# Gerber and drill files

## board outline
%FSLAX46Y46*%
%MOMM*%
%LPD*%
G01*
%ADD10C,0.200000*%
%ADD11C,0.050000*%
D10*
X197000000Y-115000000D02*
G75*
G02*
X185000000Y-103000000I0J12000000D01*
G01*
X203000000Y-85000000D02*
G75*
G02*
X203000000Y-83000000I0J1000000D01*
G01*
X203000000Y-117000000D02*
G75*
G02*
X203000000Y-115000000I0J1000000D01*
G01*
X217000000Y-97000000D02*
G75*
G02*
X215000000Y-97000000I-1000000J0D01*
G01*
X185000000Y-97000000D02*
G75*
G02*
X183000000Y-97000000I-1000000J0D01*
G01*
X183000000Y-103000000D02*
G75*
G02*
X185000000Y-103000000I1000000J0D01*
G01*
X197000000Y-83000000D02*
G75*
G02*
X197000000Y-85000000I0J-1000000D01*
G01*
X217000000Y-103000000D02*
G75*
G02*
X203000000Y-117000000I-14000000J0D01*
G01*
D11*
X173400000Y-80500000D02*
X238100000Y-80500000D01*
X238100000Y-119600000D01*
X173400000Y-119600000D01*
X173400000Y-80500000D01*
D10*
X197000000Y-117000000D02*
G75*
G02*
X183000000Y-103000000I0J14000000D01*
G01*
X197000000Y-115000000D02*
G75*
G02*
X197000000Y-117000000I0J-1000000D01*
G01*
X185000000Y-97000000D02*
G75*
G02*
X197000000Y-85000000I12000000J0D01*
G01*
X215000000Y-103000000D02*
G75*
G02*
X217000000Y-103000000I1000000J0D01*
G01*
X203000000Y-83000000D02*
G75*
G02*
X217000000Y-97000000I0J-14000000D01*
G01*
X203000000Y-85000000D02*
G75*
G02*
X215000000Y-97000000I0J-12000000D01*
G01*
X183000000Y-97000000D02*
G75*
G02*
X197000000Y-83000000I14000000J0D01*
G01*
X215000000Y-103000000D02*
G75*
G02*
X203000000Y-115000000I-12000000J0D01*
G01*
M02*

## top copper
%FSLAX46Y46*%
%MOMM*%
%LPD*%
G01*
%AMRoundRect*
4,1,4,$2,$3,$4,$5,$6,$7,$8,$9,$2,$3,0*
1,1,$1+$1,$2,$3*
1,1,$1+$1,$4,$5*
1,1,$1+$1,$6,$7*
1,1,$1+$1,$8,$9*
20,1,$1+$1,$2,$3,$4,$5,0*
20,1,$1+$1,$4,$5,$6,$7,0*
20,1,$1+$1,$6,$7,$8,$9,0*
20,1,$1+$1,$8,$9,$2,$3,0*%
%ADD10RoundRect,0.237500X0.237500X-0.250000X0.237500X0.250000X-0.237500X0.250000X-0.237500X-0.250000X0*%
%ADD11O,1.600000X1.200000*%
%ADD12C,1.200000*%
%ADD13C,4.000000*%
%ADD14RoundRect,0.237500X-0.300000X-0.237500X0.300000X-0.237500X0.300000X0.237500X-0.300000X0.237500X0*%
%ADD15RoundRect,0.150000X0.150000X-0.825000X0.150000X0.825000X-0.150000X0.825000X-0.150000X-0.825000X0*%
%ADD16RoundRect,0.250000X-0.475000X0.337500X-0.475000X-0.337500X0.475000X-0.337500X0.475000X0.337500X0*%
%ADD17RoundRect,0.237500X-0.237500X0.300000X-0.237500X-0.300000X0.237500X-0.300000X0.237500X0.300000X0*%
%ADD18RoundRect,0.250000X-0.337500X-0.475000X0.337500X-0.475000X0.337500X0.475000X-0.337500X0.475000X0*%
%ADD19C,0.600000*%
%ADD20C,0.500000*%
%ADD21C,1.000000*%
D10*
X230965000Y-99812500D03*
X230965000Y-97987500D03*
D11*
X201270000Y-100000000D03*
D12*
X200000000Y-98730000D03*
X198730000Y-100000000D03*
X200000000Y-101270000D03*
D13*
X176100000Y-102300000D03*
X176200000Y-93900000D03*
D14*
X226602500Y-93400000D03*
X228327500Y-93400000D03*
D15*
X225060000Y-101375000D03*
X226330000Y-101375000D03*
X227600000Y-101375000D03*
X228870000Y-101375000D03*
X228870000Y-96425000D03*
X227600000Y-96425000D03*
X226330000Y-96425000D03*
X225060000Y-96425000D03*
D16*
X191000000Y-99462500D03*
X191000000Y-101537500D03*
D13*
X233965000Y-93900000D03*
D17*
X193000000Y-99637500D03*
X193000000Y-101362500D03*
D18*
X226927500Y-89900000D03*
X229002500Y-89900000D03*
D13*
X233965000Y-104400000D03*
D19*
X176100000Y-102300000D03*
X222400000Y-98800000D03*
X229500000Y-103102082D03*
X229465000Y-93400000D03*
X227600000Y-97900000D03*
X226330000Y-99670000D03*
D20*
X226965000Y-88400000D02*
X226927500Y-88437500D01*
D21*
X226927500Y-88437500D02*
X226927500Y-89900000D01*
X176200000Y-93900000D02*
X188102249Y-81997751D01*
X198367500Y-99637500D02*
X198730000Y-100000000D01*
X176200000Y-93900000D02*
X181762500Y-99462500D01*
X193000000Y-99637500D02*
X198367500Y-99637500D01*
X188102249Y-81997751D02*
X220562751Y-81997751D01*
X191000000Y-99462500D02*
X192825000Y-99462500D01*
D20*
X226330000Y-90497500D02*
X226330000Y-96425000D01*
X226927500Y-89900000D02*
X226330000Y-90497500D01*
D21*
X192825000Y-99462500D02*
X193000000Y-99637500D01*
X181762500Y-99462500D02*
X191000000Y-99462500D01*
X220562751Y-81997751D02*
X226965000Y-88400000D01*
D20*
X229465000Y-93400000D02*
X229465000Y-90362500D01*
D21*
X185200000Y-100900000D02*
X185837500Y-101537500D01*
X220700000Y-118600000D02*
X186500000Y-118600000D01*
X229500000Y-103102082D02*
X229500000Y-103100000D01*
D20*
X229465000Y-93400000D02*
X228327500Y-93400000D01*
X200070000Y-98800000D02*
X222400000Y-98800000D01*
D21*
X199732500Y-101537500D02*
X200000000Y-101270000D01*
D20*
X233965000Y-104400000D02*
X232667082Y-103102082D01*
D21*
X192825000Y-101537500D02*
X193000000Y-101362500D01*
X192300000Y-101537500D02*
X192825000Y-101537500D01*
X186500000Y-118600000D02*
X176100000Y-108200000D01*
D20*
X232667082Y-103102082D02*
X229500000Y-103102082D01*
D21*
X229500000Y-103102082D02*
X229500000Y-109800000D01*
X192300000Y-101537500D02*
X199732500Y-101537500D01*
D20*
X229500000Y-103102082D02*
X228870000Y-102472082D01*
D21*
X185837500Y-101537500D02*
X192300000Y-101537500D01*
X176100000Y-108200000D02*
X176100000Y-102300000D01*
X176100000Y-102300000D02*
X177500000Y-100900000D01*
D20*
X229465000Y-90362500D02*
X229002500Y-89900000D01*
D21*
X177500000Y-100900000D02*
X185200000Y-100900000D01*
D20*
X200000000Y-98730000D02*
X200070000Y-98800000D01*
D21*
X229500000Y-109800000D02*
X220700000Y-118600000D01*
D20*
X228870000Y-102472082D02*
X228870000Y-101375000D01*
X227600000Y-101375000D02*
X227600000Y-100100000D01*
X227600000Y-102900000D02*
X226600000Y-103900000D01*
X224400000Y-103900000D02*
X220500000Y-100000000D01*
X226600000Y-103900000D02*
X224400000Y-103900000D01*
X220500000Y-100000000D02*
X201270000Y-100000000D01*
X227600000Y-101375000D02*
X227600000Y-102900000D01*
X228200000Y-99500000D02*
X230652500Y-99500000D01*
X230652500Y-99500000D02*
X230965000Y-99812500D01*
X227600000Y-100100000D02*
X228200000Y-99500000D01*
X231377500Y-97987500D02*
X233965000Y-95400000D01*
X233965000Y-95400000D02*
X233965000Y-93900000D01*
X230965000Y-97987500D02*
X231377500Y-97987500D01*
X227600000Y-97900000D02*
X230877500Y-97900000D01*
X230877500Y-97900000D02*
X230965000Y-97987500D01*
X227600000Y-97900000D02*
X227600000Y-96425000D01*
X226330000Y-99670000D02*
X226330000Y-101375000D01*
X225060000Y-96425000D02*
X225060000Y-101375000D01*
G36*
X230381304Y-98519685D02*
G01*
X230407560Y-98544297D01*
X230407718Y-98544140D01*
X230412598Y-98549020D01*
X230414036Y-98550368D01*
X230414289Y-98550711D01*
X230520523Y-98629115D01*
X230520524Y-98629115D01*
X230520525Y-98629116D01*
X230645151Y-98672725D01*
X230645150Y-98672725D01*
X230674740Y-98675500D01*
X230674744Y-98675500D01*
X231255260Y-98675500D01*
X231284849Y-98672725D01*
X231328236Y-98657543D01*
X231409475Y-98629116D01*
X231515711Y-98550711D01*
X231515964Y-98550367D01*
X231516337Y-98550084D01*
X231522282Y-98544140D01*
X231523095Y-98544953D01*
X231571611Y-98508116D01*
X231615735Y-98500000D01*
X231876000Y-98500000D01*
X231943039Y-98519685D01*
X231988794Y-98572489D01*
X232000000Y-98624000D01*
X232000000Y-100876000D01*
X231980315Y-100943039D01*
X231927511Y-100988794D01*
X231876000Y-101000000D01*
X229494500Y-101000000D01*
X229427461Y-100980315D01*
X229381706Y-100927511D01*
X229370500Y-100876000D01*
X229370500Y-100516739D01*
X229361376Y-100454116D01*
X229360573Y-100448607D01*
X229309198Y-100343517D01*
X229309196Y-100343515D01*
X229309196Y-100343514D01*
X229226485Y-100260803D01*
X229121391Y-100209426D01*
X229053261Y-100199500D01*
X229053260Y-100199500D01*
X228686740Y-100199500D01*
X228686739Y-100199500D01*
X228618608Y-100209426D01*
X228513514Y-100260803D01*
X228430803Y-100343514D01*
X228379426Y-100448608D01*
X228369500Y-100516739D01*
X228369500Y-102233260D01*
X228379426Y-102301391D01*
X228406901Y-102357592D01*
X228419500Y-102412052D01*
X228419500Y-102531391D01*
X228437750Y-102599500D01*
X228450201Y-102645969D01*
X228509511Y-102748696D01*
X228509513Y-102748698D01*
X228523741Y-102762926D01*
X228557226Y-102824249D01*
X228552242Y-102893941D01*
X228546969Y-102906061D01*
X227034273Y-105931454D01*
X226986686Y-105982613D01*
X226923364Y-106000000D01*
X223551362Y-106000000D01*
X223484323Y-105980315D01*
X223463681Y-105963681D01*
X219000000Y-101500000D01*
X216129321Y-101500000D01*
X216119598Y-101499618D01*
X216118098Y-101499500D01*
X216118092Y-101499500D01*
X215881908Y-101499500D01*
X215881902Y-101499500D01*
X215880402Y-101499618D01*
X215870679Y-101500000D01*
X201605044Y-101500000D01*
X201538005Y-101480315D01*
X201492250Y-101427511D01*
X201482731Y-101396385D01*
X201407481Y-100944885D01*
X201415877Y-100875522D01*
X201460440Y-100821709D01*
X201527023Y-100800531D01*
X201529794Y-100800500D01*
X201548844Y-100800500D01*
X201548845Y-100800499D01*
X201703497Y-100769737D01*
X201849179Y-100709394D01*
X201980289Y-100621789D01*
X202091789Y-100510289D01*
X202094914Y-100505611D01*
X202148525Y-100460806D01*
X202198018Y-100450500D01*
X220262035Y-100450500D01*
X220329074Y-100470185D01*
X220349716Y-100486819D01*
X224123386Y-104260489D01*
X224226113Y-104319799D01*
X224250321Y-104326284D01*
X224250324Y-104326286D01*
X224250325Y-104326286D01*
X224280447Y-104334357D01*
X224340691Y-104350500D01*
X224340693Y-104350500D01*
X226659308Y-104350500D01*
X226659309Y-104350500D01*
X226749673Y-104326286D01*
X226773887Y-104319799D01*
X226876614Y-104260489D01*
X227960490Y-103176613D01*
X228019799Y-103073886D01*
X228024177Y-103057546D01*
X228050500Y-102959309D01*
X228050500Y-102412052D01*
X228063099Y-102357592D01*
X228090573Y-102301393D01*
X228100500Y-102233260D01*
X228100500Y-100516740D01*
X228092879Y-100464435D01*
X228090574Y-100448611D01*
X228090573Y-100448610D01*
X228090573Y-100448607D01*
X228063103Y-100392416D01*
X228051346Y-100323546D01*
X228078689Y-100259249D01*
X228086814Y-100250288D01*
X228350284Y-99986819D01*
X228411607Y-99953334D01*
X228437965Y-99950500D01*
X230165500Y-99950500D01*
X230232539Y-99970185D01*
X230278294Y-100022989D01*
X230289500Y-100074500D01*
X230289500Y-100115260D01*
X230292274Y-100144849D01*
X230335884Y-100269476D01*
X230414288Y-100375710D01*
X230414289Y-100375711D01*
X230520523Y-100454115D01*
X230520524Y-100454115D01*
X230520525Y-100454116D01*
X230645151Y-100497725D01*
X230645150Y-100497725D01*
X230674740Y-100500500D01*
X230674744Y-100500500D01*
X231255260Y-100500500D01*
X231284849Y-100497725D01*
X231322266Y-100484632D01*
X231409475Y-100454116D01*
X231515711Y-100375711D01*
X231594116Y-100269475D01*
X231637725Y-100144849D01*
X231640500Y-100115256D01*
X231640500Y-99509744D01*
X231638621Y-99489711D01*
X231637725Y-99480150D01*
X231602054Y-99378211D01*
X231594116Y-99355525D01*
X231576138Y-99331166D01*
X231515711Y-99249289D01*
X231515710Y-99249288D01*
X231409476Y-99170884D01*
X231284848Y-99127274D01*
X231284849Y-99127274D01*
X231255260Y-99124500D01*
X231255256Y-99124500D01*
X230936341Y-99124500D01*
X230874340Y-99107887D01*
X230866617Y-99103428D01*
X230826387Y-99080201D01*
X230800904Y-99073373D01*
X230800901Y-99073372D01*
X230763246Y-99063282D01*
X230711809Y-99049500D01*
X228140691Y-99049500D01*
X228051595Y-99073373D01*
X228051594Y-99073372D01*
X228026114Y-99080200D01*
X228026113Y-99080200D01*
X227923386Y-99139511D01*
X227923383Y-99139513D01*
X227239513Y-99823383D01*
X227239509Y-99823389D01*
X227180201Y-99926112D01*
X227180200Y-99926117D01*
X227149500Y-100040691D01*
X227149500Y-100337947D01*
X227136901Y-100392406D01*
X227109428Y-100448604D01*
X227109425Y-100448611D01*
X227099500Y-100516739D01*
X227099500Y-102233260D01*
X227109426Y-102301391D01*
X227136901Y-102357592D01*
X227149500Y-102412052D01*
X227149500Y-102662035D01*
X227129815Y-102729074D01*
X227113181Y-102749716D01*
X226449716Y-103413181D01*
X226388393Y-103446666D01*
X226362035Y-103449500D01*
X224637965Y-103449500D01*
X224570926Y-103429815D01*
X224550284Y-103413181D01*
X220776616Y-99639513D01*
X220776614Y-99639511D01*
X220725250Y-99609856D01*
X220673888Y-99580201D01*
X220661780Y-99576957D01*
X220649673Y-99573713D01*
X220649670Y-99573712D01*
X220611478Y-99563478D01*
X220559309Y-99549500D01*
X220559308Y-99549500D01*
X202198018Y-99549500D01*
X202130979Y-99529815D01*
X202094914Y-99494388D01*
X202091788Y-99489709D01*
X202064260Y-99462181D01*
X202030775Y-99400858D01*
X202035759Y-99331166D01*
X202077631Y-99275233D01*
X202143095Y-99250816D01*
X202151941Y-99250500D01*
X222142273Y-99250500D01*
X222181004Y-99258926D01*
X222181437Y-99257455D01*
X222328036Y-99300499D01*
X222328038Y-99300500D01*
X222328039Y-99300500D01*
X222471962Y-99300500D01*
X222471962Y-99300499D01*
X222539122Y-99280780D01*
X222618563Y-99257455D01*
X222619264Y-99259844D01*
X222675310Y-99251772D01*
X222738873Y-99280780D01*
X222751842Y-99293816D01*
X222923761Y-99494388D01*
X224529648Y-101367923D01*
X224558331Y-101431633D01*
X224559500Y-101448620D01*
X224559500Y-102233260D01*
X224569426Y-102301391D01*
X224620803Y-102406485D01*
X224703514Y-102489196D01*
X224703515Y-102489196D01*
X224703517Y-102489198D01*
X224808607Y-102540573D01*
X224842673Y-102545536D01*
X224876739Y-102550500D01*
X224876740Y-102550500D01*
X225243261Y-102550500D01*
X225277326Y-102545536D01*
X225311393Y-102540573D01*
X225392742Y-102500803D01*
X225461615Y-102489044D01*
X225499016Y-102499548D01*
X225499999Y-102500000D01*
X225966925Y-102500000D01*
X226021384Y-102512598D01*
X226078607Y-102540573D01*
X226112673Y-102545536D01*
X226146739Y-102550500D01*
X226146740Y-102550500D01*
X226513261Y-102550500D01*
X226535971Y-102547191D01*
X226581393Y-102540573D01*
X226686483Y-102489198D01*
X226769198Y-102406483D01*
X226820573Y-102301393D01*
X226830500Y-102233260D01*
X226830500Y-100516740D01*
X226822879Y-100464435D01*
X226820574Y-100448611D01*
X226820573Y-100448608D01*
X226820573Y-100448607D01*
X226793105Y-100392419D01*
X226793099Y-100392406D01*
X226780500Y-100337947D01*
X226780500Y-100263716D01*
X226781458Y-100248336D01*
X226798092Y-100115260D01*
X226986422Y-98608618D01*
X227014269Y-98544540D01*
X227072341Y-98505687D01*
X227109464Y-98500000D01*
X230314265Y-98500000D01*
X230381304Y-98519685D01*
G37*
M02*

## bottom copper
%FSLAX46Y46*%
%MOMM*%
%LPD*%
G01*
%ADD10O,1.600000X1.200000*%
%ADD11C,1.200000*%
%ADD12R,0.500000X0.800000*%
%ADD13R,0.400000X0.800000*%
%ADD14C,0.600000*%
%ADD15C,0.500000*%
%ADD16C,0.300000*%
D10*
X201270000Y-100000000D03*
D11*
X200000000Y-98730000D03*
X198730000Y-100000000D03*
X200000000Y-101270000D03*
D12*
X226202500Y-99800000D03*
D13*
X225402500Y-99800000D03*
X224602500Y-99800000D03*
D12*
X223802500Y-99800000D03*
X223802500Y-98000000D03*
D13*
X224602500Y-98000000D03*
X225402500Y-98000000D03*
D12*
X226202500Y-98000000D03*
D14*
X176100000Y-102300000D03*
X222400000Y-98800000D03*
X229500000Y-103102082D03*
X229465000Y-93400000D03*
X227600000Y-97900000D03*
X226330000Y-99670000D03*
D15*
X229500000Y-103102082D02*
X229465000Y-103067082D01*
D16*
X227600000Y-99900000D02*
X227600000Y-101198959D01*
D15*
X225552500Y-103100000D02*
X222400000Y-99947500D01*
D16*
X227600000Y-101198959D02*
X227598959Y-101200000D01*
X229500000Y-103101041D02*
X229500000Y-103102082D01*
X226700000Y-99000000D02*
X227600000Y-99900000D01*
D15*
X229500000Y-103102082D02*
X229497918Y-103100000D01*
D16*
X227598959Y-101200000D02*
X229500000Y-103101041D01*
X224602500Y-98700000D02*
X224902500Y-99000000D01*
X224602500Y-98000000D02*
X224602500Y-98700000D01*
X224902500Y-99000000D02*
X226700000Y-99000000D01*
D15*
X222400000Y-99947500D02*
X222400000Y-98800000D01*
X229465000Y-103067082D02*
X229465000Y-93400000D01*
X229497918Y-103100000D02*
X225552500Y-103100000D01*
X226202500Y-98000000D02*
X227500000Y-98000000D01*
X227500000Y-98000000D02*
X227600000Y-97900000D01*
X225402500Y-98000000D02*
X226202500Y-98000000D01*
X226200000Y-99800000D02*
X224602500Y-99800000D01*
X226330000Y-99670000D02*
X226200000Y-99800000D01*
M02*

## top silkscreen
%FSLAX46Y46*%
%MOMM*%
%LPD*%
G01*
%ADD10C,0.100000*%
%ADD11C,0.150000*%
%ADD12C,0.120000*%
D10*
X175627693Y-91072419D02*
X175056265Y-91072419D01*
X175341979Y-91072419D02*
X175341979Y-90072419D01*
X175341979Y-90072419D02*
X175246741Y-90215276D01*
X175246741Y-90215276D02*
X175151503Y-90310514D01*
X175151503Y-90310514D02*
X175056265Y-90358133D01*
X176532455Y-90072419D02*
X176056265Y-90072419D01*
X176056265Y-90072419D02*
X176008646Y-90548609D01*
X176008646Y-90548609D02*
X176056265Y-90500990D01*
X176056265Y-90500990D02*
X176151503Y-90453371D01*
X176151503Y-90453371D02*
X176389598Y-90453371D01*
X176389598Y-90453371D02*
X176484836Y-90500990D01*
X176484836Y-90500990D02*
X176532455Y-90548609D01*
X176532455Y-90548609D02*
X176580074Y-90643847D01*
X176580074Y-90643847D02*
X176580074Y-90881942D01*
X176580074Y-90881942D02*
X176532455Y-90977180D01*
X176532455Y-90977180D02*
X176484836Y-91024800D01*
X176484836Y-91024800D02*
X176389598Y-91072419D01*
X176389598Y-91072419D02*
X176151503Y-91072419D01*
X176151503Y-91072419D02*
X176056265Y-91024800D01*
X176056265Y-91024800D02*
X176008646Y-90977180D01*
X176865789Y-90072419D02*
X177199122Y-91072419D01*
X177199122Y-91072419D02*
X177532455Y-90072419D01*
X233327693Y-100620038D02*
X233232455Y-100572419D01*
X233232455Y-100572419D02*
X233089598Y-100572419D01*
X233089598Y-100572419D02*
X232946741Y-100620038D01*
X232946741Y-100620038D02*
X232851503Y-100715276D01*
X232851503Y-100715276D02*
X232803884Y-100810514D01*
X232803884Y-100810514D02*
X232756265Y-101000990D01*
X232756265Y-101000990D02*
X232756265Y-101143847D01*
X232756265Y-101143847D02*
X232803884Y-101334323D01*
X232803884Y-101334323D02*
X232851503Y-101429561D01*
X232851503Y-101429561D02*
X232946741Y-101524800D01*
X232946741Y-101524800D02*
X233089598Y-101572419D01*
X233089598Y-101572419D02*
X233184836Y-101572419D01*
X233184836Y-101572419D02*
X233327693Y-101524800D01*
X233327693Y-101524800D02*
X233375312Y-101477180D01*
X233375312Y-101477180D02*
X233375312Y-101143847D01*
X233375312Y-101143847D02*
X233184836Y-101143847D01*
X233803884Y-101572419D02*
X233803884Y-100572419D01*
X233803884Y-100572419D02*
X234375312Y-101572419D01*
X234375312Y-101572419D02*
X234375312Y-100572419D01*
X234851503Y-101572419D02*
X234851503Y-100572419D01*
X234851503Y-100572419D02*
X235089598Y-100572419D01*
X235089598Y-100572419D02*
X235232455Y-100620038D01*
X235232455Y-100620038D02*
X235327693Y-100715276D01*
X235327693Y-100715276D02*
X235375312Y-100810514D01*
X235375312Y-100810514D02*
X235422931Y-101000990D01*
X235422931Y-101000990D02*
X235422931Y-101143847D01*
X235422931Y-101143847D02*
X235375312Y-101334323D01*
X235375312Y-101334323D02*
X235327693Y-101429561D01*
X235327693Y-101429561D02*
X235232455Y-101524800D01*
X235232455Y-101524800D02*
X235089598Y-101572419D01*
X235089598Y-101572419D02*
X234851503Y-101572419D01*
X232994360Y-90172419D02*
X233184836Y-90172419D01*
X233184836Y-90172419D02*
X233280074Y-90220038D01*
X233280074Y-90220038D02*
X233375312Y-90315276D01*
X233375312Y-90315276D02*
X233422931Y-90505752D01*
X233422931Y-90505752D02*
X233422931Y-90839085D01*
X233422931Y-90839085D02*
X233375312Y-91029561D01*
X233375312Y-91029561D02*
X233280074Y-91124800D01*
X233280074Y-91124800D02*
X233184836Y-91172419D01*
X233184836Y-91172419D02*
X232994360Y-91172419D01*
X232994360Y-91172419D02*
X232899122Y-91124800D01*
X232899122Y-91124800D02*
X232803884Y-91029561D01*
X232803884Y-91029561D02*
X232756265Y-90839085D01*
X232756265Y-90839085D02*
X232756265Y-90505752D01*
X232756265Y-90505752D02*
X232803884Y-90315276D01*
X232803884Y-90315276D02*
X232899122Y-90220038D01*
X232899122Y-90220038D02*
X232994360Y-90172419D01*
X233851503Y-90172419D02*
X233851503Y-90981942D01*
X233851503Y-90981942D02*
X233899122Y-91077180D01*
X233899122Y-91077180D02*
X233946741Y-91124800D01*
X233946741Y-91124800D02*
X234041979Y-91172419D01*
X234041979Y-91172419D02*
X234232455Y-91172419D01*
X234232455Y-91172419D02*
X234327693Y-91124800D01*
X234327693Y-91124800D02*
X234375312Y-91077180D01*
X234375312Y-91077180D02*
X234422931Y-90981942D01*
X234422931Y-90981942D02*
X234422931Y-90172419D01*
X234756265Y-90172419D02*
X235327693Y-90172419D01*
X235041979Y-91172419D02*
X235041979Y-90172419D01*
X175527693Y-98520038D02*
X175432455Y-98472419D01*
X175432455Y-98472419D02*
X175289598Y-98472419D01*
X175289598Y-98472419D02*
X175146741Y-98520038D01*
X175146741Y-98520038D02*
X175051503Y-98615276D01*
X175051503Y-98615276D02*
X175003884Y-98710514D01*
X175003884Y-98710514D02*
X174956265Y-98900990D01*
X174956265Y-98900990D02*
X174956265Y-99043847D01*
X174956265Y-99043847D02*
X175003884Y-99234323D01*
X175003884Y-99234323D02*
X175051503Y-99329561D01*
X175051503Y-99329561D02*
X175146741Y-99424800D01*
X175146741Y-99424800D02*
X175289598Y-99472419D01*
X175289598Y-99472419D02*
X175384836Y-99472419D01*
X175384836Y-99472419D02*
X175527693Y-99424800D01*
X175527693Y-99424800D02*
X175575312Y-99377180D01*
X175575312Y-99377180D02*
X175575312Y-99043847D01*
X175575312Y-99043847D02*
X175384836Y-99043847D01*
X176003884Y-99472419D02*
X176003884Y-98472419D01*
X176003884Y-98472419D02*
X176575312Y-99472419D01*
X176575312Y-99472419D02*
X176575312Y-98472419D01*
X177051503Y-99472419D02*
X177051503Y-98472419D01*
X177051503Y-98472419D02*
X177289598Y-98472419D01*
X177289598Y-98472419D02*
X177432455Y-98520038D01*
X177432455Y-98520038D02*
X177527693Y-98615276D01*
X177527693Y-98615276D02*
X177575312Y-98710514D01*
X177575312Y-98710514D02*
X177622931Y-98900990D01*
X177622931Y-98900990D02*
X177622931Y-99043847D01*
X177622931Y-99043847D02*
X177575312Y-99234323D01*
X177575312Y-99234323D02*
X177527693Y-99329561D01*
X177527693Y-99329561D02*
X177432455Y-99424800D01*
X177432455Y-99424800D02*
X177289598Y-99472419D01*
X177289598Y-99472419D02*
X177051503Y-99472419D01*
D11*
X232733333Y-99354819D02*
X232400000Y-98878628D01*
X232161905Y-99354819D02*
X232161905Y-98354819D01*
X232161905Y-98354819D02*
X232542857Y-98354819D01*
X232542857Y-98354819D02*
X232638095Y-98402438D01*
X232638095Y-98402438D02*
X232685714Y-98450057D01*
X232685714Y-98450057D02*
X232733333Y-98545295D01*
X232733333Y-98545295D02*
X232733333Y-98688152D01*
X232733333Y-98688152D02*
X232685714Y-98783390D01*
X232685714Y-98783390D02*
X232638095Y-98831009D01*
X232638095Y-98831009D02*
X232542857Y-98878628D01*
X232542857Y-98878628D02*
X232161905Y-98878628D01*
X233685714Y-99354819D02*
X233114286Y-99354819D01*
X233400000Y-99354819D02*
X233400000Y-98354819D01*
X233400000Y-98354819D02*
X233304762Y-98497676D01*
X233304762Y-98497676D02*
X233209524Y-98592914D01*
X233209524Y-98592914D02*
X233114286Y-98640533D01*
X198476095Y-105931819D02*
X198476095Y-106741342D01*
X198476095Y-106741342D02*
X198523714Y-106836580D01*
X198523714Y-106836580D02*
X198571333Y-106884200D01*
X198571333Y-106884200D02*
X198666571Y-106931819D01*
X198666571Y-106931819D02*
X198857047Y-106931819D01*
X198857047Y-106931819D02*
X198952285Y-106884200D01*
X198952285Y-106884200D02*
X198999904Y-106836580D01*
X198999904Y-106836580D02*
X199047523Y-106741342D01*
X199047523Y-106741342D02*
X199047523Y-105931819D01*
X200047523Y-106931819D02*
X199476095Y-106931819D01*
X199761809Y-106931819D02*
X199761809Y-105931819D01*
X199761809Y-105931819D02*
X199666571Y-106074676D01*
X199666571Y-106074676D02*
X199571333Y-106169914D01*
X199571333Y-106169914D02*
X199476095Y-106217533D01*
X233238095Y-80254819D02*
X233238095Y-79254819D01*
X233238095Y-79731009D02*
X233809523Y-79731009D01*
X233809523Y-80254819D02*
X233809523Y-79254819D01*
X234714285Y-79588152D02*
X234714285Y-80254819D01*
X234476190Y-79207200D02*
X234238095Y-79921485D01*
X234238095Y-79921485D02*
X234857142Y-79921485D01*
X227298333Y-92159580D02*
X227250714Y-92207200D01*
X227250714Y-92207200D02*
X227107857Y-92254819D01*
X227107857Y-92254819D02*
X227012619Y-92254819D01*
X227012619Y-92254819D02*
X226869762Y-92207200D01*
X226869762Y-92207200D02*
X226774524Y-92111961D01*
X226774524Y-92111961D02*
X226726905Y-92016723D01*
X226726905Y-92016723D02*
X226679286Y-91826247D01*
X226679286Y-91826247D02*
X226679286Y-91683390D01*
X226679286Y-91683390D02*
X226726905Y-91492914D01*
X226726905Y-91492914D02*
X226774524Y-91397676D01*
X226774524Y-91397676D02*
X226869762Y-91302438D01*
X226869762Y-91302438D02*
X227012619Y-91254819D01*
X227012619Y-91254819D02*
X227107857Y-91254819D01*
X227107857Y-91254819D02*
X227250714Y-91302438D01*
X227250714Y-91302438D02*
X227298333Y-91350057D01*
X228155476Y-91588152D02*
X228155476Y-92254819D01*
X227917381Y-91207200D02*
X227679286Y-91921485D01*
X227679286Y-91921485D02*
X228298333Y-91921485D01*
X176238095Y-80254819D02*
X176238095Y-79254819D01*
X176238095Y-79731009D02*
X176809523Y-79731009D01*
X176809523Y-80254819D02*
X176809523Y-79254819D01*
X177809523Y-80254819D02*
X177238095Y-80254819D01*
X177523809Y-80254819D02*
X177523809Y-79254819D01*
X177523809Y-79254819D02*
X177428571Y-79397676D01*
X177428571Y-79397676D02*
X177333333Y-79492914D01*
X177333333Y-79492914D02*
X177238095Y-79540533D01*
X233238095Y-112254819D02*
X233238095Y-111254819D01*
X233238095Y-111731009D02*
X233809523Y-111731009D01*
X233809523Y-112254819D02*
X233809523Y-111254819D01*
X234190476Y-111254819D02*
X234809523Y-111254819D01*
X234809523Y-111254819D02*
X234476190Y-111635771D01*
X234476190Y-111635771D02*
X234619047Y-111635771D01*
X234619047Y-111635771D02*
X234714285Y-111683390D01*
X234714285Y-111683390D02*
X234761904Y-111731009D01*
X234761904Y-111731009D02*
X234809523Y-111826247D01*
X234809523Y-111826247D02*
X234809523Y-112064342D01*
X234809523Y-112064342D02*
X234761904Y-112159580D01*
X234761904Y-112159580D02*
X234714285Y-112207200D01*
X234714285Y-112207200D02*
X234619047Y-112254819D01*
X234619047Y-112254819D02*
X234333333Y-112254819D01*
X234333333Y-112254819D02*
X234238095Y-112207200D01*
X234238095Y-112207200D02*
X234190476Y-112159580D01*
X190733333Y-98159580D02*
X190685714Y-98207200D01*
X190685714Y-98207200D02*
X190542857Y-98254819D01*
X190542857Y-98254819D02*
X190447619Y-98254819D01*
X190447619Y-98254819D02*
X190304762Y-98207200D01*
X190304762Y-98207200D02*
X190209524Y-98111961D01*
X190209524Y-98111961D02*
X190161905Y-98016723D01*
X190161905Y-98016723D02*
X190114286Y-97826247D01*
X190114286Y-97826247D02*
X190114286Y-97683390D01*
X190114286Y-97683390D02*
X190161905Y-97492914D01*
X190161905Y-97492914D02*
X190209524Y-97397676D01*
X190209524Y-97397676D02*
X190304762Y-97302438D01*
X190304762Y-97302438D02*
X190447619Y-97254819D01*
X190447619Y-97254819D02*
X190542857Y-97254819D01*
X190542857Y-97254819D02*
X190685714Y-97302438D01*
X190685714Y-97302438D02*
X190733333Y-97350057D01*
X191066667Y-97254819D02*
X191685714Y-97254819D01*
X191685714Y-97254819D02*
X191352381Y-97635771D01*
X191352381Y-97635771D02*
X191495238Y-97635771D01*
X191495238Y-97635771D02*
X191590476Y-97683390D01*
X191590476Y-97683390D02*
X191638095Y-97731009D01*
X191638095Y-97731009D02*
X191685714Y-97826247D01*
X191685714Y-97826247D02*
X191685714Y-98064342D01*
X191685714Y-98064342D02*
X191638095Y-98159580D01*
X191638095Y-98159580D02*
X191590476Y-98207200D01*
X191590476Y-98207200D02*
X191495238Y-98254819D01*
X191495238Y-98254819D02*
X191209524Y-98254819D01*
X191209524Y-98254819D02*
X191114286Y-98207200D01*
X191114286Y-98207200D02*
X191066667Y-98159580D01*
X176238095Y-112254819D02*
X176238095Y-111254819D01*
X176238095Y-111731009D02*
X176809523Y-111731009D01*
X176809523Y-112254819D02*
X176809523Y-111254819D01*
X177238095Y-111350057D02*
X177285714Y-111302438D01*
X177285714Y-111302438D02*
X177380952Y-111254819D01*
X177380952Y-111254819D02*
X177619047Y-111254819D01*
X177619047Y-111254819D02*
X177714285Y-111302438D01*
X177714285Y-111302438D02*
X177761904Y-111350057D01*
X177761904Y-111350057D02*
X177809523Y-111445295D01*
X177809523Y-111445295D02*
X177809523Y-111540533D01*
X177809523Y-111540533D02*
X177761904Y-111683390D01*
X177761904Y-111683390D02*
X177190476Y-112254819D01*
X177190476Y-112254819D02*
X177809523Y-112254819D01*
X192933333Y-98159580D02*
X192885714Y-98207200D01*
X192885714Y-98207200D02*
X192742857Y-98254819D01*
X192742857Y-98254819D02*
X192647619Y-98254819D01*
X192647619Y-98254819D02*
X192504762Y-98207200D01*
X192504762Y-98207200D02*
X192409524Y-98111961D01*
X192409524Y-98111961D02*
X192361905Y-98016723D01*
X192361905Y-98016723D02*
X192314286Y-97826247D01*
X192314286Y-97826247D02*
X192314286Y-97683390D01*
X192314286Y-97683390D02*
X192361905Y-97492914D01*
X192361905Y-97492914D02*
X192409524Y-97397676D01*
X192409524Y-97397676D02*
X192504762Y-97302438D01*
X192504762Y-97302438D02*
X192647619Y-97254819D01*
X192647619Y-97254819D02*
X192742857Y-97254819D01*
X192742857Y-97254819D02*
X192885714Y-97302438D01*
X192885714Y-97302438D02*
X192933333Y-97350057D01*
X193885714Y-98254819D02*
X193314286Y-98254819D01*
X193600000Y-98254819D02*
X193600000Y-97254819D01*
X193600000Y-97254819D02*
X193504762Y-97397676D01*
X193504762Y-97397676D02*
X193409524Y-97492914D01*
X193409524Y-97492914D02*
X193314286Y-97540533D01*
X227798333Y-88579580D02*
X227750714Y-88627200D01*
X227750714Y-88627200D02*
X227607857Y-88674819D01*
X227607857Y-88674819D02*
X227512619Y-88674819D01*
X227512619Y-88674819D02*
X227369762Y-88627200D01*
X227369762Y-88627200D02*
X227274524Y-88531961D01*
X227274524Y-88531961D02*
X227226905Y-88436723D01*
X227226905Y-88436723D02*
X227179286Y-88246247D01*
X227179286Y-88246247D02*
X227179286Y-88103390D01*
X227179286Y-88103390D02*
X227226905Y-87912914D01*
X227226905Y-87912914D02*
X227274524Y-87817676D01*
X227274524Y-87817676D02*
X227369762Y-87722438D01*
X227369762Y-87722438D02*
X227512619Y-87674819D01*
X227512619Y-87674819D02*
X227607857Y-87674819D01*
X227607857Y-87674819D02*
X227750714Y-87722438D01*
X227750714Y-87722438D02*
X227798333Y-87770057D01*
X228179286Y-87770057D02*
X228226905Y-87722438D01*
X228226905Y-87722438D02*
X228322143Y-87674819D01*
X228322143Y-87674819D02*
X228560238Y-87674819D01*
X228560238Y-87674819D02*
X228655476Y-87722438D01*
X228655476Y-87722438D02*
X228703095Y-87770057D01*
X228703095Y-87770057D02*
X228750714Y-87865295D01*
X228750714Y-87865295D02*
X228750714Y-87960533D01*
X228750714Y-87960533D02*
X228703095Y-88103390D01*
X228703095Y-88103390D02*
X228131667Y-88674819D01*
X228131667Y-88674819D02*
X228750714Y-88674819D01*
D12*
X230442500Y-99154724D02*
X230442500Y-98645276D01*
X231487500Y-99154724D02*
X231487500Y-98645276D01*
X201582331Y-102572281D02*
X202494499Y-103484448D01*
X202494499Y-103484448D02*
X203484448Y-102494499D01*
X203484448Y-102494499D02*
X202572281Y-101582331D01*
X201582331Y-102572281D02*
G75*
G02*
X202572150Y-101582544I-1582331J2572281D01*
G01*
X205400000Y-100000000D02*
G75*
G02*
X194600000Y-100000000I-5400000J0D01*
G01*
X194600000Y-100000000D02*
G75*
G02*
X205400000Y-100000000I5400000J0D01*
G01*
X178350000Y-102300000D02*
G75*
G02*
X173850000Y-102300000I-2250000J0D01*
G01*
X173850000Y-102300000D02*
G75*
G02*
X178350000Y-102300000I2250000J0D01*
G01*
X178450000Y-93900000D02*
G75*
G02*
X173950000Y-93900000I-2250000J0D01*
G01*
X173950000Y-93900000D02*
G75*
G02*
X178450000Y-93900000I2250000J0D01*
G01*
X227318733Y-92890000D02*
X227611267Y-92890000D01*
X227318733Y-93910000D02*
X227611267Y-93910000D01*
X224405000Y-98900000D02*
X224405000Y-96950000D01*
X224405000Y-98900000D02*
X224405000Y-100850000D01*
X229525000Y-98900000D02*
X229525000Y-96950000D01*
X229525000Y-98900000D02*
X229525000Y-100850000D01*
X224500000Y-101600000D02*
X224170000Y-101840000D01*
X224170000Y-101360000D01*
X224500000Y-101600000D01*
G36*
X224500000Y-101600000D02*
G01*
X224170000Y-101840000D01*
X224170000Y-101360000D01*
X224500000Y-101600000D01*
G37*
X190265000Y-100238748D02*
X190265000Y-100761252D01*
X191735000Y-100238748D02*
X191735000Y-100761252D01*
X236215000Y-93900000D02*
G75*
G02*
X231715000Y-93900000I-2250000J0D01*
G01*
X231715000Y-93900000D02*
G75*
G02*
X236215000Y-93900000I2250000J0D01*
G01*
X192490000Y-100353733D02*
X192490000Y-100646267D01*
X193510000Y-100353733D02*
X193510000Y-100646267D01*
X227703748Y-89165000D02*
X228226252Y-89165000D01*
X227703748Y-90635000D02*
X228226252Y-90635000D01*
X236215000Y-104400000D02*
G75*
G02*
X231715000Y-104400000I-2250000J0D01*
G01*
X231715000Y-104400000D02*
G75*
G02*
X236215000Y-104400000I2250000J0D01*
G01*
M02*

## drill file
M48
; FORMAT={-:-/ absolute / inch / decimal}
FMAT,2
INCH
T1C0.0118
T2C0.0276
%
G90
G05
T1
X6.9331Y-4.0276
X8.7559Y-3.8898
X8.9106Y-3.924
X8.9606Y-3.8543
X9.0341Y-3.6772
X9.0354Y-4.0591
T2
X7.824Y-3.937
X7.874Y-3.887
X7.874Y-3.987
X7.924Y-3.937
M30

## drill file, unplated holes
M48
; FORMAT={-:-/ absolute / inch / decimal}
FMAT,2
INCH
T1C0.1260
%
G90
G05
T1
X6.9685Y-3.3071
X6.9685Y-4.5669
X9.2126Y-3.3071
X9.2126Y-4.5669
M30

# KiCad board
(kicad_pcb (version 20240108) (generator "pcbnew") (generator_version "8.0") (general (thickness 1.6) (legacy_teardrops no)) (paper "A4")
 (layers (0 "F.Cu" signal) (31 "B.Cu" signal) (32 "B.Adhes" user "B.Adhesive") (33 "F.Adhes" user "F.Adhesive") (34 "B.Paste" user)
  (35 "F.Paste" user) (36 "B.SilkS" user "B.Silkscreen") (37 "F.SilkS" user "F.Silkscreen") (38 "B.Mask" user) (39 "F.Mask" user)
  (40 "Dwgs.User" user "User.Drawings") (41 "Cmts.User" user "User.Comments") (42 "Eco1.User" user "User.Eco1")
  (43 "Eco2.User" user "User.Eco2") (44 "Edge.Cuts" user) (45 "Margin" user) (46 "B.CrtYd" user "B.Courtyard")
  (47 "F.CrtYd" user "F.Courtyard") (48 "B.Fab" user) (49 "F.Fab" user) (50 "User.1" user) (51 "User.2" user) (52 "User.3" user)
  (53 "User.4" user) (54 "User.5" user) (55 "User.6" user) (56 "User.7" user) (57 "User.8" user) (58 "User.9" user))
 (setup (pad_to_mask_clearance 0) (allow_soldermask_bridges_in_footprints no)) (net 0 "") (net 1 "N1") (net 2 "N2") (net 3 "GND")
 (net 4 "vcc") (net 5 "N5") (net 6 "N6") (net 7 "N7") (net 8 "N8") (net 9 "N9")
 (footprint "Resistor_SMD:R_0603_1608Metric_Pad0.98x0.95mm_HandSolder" (layer "F.Cu") (at 230.965 98.9 90)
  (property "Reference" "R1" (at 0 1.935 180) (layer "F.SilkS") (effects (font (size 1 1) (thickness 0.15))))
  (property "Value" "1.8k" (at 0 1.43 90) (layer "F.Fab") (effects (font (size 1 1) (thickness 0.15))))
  (fp_line (start -0.254724 -0.5225) (end 0.254724 -0.5225) (stroke (width 0.12) (type solid)) (layer "F.SilkS"))
  (fp_line (start -0.254724 0.5225) (end 0.254724 0.5225) (stroke (width 0.12) (type solid)) (layer "F.SilkS"))
  (pad "1" smd roundrect (at -0.9125 0 90) (size 0.975 0.95) (layers "F.Cu" "F.Paste" "F.Mask") (roundrect_rratio 0.25) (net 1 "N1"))
  (pad "2" smd roundrect (at 0.9125 0 90) (size 0.975 0.95) (layers "F.Cu" "F.Paste" "F.Mask") (roundrect_rratio 0.25) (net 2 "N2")))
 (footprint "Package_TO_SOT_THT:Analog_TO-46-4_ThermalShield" (layer "F.Cu") (at 201.27 100 180)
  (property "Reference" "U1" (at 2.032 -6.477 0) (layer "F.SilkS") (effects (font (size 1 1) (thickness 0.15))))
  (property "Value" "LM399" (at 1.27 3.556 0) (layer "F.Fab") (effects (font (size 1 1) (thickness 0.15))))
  (fp_line (start -0.312331 -2.572281) (end -1.224499 -3.484448) (stroke (width 0.12) (type solid)) (layer "F.SilkS"))
  (fp_line (start -1.224499 -3.484448) (end -2.214448 -2.494499) (stroke (width 0.12) (type solid)) (layer "F.SilkS"))
  (fp_line (start -2.214448 -2.494499) (end -1.302281 -1.582331) (stroke (width 0.12) (type solid)) (layer "F.SilkS"))
  (fp_arc (start -0.312331 -2.572281) (mid 3.405374 2.135551) (end -1.30215 -1.582544) (stroke (width 0.12) (type solid)) (layer "F.SilkS"))
  (fp_circle (center 1.27 0) (end 6.67 0) (stroke (width 0.12) (type solid)) (fill none) (layer "F.SilkS"))
  (pad "1" thru_hole oval (at 0 0 180) (size 1.6 1.2) (drill 0.7) (layers "*.Cu" "*.Mask") (remove_unused_layers no) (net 1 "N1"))
  (pad "2" thru_hole circle (at 1.27 1.27 180) (size 1.2 1.2) (drill 0.7) (layers "*.Cu" "*.Mask") (remove_unused_layers no) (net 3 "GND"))
  (pad "3" thru_hole circle (at 2.54 0 180) (size 1.2 1.2) (drill 0.7) (layers "*.Cu" "*.Mask") (remove_unused_layers no) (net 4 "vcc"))
  (pad "4" thru_hole circle (at 1.27 -1.27 180) (size 1.2 1.2) (drill 0.7) (layers "*.Cu" "*.Mask") (remove_unused_layers no) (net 3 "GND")))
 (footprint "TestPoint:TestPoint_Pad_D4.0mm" (layer "F.Cu") (at 176.1 102.3)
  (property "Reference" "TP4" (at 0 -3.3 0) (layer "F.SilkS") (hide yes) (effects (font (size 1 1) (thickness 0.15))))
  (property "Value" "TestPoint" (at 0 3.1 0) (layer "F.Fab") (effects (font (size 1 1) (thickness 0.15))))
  (fp_circle (center 0 0) (end 0 2.25) (stroke (width 0.12) (type solid)) (fill none) (layer "F.SilkS"))
  (pad "1" smd circle (at 0 0) (size 4 4) (layers "F.Cu" "F.Mask") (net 3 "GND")))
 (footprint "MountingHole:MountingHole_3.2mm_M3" (layer "F.Cu") (at 234 84)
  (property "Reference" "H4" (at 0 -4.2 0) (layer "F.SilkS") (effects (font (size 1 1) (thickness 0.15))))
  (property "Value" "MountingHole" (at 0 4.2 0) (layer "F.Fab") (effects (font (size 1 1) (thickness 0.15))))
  (pad "" np_thru_hole circle (at 0 0) (size 3.2 3.2) (drill 3.2) (layers "*.Cu" "*.Mask")))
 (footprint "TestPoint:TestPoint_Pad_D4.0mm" (layer "F.Cu") (at 176.2 93.9)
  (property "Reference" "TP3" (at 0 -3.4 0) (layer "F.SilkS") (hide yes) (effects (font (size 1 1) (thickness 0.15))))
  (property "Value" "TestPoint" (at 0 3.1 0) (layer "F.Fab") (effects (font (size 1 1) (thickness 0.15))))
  (fp_circle (center 0 0) (end 0 2.25) (stroke (width 0.12) (type solid)) (fill none) (layer "F.SilkS"))
  (pad "1" smd circle (at 0 0) (size 4 4) (layers "F.Cu" "F.Mask") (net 4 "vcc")))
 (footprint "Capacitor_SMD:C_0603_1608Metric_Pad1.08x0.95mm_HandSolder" (layer "F.Cu") (at 227.465 93.4)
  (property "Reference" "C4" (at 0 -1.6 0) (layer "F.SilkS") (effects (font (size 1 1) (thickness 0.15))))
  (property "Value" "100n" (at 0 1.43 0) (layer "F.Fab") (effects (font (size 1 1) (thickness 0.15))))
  (fp_line (start -0.146267 -0.51) (end 0.146267 -0.51) (stroke (width 0.12) (type solid)) (layer "F.SilkS"))
  (fp_line (start -0.146267 0.51) (end 0.146267 0.51) (stroke (width 0.12) (type solid)) (layer "F.SilkS"))
  (pad "1" smd roundrect (at -0.8625 0) (size 1.075 0.95) (layers "F.Cu" "F.Paste" "F.Mask") (roundrect_rratio 0.25) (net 4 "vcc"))
  (pad "2" smd roundrect (at 0.8625 0) (size 1.075 0.95) (layers "F.Cu" "F.Paste" "F.Mask") (roundrect_rratio 0.25) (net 3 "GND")))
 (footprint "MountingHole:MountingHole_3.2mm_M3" (layer "F.Cu") (at 177 84)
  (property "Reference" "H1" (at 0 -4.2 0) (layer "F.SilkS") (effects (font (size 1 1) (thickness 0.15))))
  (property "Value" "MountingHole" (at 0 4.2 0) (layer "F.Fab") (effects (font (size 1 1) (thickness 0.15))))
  (pad "" np_thru_hole circle (at 0 0) (size 3.2 3.2) (drill 3.2) (layers "*.Cu" "*.Mask")))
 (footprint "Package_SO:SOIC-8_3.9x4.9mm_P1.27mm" (layer "F.Cu") (at 226.965 98.9 90)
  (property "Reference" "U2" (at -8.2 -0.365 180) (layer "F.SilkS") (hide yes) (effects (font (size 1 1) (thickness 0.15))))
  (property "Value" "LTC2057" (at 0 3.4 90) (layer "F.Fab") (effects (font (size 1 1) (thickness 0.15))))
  (fp_line (start 0 -2.56) (end 1.95 -2.56) (stroke (width 0.12) (type solid)) (layer "F.SilkS"))
  (fp_line (start 0 -2.56) (end -1.95 -2.56) (stroke (width 0.12) (type solid)) (layer "F.SilkS"))
  (fp_line (start 0 2.56) (end 1.95 2.56) (stroke (width 0.12) (type solid)) (layer "F.SilkS"))
  (fp_line (start 0 2.56) (end -1.95 2.56) (stroke (width 0.12) (type solid)) (layer "F.SilkS"))
  (fp_poly
   (pts (xy -2.7 -2.465) (xy -2.94 -2.795) (xy -2.46 -2.795) (xy -2.7 -2.465)) (stroke (width 0.12) (type solid)) (fill solid)
   (layer "F.SilkS"))
  (pad "1" smd roundrect (at -2.475 -1.905 90) (size 1.95 0.6) (layers "F.Cu" "F.Paste" "F.Mask") (roundrect_rratio 0.25) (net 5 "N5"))
  (pad "2" smd roundrect (at -2.475 -0.635 90) (size 1.95 0.6) (layers "F.Cu" "F.Paste" "F.Mask") (roundrect_rratio 0.25) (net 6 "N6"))
  (pad "3" smd roundrect (at -2.475 0.635 90) (size 1.95 0.6) (layers "F.Cu" "F.Paste" "F.Mask") (roundrect_rratio 0.25) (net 1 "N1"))
  (pad "4" smd roundrect (at -2.475 1.905 90) (size 1.95 0.6) (layers "F.Cu" "F.Paste" "F.Mask") (roundrect_rratio 0.25) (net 3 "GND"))
  (pad "5" smd roundrect (at 2.475 1.905 90) (size 1.95 0.6) (layers "F.Cu" "F.Paste" "F.Mask") (roundrect_rratio 0.25) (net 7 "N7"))
  (pad "6" smd roundrect (at 2.475 0.635 90) (size 1.95 0.6) (layers "F.Cu" "F.Paste" "F.Mask") (roundrect_rratio 0.25) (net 2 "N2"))
  (pad "7" smd roundrect (at 2.475 -0.635 90) (size 1.95 0.6) (layers "F.Cu" "F.Paste" "F.Mask") (roundrect_rratio 0.25) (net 4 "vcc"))
  (pad "8" smd roundrect (at 2.475 -1.905 90) (size 1.95 0.6) (layers "F.Cu" "F.Paste" "F.Mask") (roundrect_rratio 0.25) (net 5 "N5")))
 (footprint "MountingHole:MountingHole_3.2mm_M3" (layer "F.Cu") (at 234 116)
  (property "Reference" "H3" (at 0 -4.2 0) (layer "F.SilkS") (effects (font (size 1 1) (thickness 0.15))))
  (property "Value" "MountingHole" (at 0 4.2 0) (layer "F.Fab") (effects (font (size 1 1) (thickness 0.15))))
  (pad "" np_thru_hole circle (at 0 0) (size 3.2 3.2) (drill 3.2) (layers "*.Cu" "*.Mask")))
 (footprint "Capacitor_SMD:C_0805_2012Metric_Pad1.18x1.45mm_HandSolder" (layer "F.Cu") (at 191 100.5 -90)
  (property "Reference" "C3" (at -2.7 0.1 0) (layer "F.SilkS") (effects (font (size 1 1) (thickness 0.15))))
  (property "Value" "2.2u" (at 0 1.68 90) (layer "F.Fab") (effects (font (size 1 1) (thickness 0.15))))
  (fp_line (start -0.261252 0.735) (end 0.261252 0.735) (stroke (width 0.12) (type solid)) (layer "F.SilkS"))
  (fp_line (start -0.261252 -0.735) (end 0.261252 -0.735) (stroke (width 0.12) (type solid)) (layer "F.SilkS"))
  (pad "1" smd roundrect (at -1.0375 0 270) (size 1.175 1.45) (layers "F.Cu" "F.Paste" "F.Mask") (roundrect_rratio 0.212766) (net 4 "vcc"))
  (pad "2" smd roundrect (at 1.0375 0 270) (size 1.175 1.45) (layers "F.Cu" "F.Paste" "F.Mask") (roundrect_rratio 0.212766) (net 3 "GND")))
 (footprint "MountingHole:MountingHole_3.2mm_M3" (layer "F.Cu") (at 177 116)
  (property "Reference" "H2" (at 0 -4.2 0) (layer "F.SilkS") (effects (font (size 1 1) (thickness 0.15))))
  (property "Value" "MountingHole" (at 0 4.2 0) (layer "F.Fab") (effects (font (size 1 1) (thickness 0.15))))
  (pad "" np_thru_hole circle (at 0 0) (size 3.2 3.2) (drill 3.2) (layers "*.Cu" "*.Mask")))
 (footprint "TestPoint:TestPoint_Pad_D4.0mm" (layer "F.Cu") (at 233.965 93.9)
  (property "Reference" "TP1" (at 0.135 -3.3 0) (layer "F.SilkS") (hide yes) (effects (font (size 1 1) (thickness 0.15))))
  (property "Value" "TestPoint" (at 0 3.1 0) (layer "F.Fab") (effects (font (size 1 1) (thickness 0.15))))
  (fp_circle (center 0 0) (end 0 2.25) (stroke (width 0.12) (type solid)) (fill none) (layer "F.SilkS"))
  (pad "1" smd circle (at 0 0) (size 4 4) (layers "F.Cu" "F.Mask") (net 2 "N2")))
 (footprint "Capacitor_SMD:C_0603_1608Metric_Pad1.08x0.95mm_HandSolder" (layer "F.Cu") (at 193 100.5 -90)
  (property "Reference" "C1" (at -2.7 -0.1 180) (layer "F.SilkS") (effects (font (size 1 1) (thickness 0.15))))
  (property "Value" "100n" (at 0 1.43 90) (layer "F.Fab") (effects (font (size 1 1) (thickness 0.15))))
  (fp_line (start -0.146267 0.51) (end 0.146267 0.51) (stroke (width 0.12) (type solid)) (layer "F.SilkS"))
  (fp_line (start -0.146267 -0.51) (end 0.146267 -0.51) (stroke (width 0.12) (type solid)) (layer "F.SilkS"))
  (pad "1" smd roundrect (at -0.8625 0 270) (size 1.075 0.95) (layers "F.Cu" "F.Paste" "F.Mask") (roundrect_rratio 0.25) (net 4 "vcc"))
  (pad "2" smd roundrect (at 0.8625 0 270) (size 1.075 0.95) (layers "F.Cu" "F.Paste" "F.Mask") (roundrect_rratio 0.25) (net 3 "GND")))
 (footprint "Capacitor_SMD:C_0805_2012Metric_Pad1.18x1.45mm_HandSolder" (layer "F.Cu") (at 227.965 89.9)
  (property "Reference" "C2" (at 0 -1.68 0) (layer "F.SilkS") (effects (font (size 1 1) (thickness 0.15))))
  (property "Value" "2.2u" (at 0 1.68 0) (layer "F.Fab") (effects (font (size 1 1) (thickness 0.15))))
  (fp_line (start -0.261252 -0.735) (end 0.261252 -0.735) (stroke (width 0.12) (type solid)) (layer "F.SilkS"))
  (fp_line (start -0.261252 0.735) (end 0.261252 0.735) (stroke (width 0.12) (type solid)) (layer "F.SilkS"))
  (pad "1" smd roundrect (at -1.0375 0) (size 1.175 1.45) (layers "F.Cu" "F.Paste" "F.Mask") (roundrect_rratio 0.212766) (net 4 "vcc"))
  (pad "2" smd roundrect (at 1.0375 0) (size 1.175 1.45) (layers "F.Cu" "F.Paste" "F.Mask") (roundrect_rratio 0.212766) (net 3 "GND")))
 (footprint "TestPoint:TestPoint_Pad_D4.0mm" (layer "F.Cu") (at 233.965 104.4)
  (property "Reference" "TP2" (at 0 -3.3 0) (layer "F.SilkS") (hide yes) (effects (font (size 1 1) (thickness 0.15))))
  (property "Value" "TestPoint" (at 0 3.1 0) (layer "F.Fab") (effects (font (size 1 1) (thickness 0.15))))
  (fp_circle (center 0 0) (end 0 2.25) (stroke (width 0.12) (type solid)) (fill none) (layer "F.SilkS"))
  (pad "1" smd circle (at 0 0) (size 4 4) (layers "F.Cu" "F.Mask") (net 3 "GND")))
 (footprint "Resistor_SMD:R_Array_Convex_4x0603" (layer "B.Cu") (at 225.0025 98.9 90)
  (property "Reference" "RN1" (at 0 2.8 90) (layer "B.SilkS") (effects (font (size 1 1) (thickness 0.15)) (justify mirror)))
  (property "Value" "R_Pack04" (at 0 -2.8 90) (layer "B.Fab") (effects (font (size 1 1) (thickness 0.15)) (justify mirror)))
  (pad "1" smd rect (at -0.9 1.2 90) (size 0.8 0.5) (layers "B.Cu" "B.Paste" "B.Mask") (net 6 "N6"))
  (pad "2" smd rect (at -0.9 0.4 90) (size 0.8 0.4) (layers "B.Cu" "B.Paste" "B.Mask") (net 6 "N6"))
  (pad "3" smd rect (at -0.9 -0.4 90) (size 0.8 0.4) (layers "B.Cu" "B.Paste" "B.Mask") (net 6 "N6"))
  (pad "4" smd rect (at -0.9 -1.2 90) (size 0.8 0.5) (layers "B.Cu" "B.Paste" "B.Mask") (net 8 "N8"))
  (pad "5" smd rect (at 0.9 -1.2 90) (size 0.8 0.5) (layers "B.Cu" "B.Paste" "B.Mask") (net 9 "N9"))
  (pad "6" smd rect (at 0.9 -0.4 90) (size 0.8 0.4) (layers "B.Cu" "B.Paste" "B.Mask") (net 3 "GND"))
  (pad "7" smd rect (at 0.9 0.4 90) (size 0.8 0.4) (layers "B.Cu" "B.Paste" "B.Mask") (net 2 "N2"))
  (pad "8" smd rect (at 0.9 1.2 90) (size 0.8 0.5) (layers "B.Cu" "B.Paste" "B.Mask") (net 2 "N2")))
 (gr_arc (start 197 115) (mid 188.514719 111.485281) (end 185 103) (stroke (width 0.2) (type default)) (layer "Edge.Cuts"))
 (gr_arc (start 203 85) (mid 202 84) (end 203 83) (stroke (width 0.2) (type default)) (layer "Edge.Cuts"))
 (gr_arc (start 203 117) (mid 202 116) (end 203 115) (stroke (width 0.2) (type default)) (layer "Edge.Cuts"))
 (gr_arc (start 217 97) (mid 216 98) (end 215 97) (stroke (width 0.2) (type default)) (layer "Edge.Cuts"))
 (gr_arc (start 185 97) (mid 184 98) (end 183 97) (stroke (width 0.2) (type default)) (layer "Edge.Cuts"))
 (gr_arc (start 183 103) (mid 184 102) (end 185 103) (stroke (width 0.2) (type default)) (layer "Edge.Cuts"))
 (gr_arc (start 197 83) (mid 198 84) (end 197 85) (stroke (width 0.2) (type default)) (layer "Edge.Cuts"))
 (gr_arc (start 217 103) (mid 212.899495 112.899495) (end 203 117) (stroke (width 0.2) (type default)) (layer "Edge.Cuts"))
 (gr_rect (start 173.4 80.5) (end 238.1 119.6) (stroke (width 0.05) (type default)) (fill none) (layer "Edge.Cuts"))
 (gr_arc (start 197 117) (mid 187.100505 112.899495) (end 183 103) (stroke (width 0.2) (type default)) (layer "Edge.Cuts"))
 (gr_arc (start 197 115) (mid 198 116) (end 197 117) (stroke (width 0.2) (type default)) (layer "Edge.Cuts"))
 (gr_arc (start 185 97) (mid 188.514719 88.514719) (end 197 85) (stroke (width 0.2) (type default)) (layer "Edge.Cuts"))
 (gr_arc (start 215 103) (mid 216 102) (end 217 103) (stroke (width 0.2) (type default)) (layer "Edge.Cuts"))
 (gr_arc (start 203 83) (mid 212.899495 87.100505) (end 217 97) (stroke (width 0.2) (type default)) (layer "Edge.Cuts"))
 (gr_arc (start 203 85) (mid 211.485281 88.514719) (end 215 97) (stroke (width 0.2) (type default)) (layer "Edge.Cuts"))
 (gr_arc (start 183 97) (mid 187.100505 87.100505) (end 197 83) (stroke (width 0.2) (type default)) (layer "Edge.Cuts"))
 (gr_arc (start 215 103) (mid 211.485281 111.485281) (end 203 115) (stroke (width 0.2) (type default)) (layer "Edge.Cuts"))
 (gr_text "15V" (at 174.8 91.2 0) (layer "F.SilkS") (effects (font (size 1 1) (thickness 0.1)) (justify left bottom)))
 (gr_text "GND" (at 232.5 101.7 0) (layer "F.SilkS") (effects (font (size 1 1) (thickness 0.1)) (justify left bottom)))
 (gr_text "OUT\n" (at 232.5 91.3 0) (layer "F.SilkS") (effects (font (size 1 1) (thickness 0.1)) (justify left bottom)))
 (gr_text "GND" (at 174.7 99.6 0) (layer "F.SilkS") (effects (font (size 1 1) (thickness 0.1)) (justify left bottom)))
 (segment (start 226.965 88.4) (end 226.9275 88.4375) (width 0.5) (layer "F.Cu") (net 4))
 (segment (start 226.9275 88.4375) (end 226.9275 89.9) (width 1) (layer "F.Cu") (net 4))
 (segment (start 176.2 93.9) (end 188.102249 81.997751) (width 1) (layer "F.Cu") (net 4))
 (segment (start 198.3675 99.6375) (end 198.73 100) (width 1) (layer "F.Cu") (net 4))
 (segment (start 176.2 93.9) (end 181.7625 99.4625) (width 1) (layer "F.Cu") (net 4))
 (segment (start 193 99.6375) (end 198.3675 99.6375) (width 1) (layer "F.Cu") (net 4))
 (segment (start 188.102249 81.997751) (end 220.562751 81.997751) (width 1) (layer "F.Cu") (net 4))
 (segment (start 191 99.4625) (end 192.825 99.4625) (width 1) (layer "F.Cu") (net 4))
 (segment (start 226.33 90.4975) (end 226.33 96.425) (width 0.5) (layer "F.Cu") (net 4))
 (segment (start 226.9275 89.9) (end 226.33 90.4975) (width 0.5) (layer "F.Cu") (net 4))
 (segment (start 192.825 99.4625) (end 193 99.6375) (width 1) (layer "F.Cu") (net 4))
 (segment (start 181.7625 99.4625) (end 191 99.4625) (width 1) (layer "F.Cu") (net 4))
 (segment (start 220.562751 81.997751) (end 226.965 88.4) (width 1) (layer "F.Cu") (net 4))
 (segment (start 229.465 93.4) (end 229.465 90.3625) (width 0.5) (layer "F.Cu") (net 3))
 (segment (start 185.2 100.9) (end 185.8375 101.5375) (width 1) (layer "F.Cu") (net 3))
 (segment (start 220.7 118.6) (end 186.5 118.6) (width 1) (layer "F.Cu") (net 3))
 (segment (start 229.5 103.102082) (end 229.5 103.1) (width 1) (layer "F.Cu") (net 3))
 (segment (start 229.465 93.4) (end 228.3275 93.4) (width 0.5) (layer "F.Cu") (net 3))
 (segment (start 200.07 98.8) (end 222.4 98.8) (width 0.5) (layer "F.Cu") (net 3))
 (segment (start 199.7325 101.5375) (end 200 101.27) (width 1) (layer "F.Cu") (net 3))
 (segment (start 233.965 104.4) (end 232.667082 103.102082) (width 0.5) (layer "F.Cu") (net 3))
 (segment (start 192.825 101.5375) (end 193 101.3625) (width 1) (layer "F.Cu") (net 3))
 (segment (start 192.3 101.5375) (end 192.825 101.5375) (width 1) (layer "F.Cu") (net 3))
 (segment (start 186.5 118.6) (end 176.1 108.2) (width 1) (layer "F.Cu") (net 3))
 (segment (start 232.667082 103.102082) (end 229.5 103.102082) (width 0.5) (layer "F.Cu") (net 3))
 (segment (start 229.5 103.102082) (end 229.5 109.8) (width 1) (layer "F.Cu") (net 3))
 (segment (start 192.3 101.5375) (end 199.7325 101.5375) (width 1) (layer "F.Cu") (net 3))
 (segment (start 229.5 103.102082) (end 228.87 102.472082) (width 0.5) (layer "F.Cu") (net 3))
 (segment (start 185.8375 101.5375) (end 192.3 101.5375) (width 1) (layer "F.Cu") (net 3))
 (segment (start 176.1 108.2) (end 176.1 102.3) (width 1) (layer "F.Cu") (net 3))
 (segment (start 176.1 102.3) (end 177.5 100.9) (width 1) (layer "F.Cu") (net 3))
 (segment (start 229.465 90.3625) (end 229.0025 89.9) (width 0.5) (layer "F.Cu") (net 3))
 (segment (start 177.5 100.9) (end 185.2 100.9) (width 1) (layer "F.Cu") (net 3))
 (segment (start 200 98.73) (end 200.07 98.8) (width 0.5) (layer "F.Cu") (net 3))
 (segment (start 229.5 109.8) (end 220.7 118.6) (width 1) (layer "F.Cu") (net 3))
 (segment (start 228.87 102.472082) (end 228.87 101.375) (width 0.5) (layer "F.Cu") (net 3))
 (via (at 176.1 102.3) (size 0.6) (drill 0.3) (layers "F.Cu" "B.Cu") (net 3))
 (via (at 222.4 98.8) (size 0.6) (drill 0.3) (layers "F.Cu" "B.Cu") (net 3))
 (via (at 229.5 103.102082) (size 0.6) (drill 0.3) (layers "F.Cu" "B.Cu") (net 3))
 (via (at 229.465 93.4) (size 0.6) (drill 0.3) (layers "F.Cu" "B.Cu") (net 3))
 (segment (start 229.5 103.102082) (end 229.465 103.067082) (width 0.5) (layer "B.Cu") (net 3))
 (segment (start 227.6 99.9) (end 227.6 101.198959) (width 0.3) (layer "B.Cu") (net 3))
 (segment (start 225.5525 103.1) (end 222.4 99.9475) (width 0.5) (layer "B.Cu") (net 3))
 (segment (start 227.6 101.198959) (end 227.598959 101.2) (width 0.3) (layer "B.Cu") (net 3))
 (segment (start 229.5 103.101041) (end 229.5 103.102082) (width 0.3) (layer "B.Cu") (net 3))
 (segment (start 226.7 99) (end 227.6 99.9) (width 0.3) (layer "B.Cu") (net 3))
 (segment (start 229.5 103.102082) (end 229.497918 103.1) (width 0.5) (layer "B.Cu") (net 3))
 (segment (start 227.598959 101.2) (end 229.5 103.101041) (width 0.3) (layer "B.Cu") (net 3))
 (segment (start 224.6025 98.7) (end 224.9025 99) (width 0.3) (layer "B.Cu") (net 3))
 (segment (start 224.6025 98) (end 224.6025 98.7) (width 0.3) (layer "B.Cu") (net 3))
 (segment (start 224.9025 99) (end 226.7 99) (width 0.3) (layer "B.Cu") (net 3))
 (segment (start 222.4 99.9475) (end 222.4 98.8) (width 0.5) (layer "B.Cu") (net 3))
 (segment (start 229.465 103.067082) (end 229.465 93.4) (width 0.5) (layer "B.Cu") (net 3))
 (segment (start 229.497918 103.1) (end 225.5525 103.1) (width 0.5) (layer "B.Cu") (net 3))
 (segment (start 227.6 101.375) (end 227.6 100.1) (width 0.5) (layer "F.Cu") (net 1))
 (segment (start 227.6 102.9) (end 226.6 103.9) (width 0.5) (layer "F.Cu") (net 1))
 (segment (start 224.4 103.9) (end 220.5 100) (width 0.5) (layer "F.Cu") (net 1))
 (segment (start 226.6 103.9) (end 224.4 103.9) (width 0.5) (layer "F.Cu") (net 1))
 (segment (start 220.5 100) (end 201.27 100) (width 0.5) (layer "F.Cu") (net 1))
 (segment (start 227.6 101.375) (end 227.6 102.9) (width 0.5) (layer "F.Cu") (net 1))
 (segment (start 228.2 99.5) (end 230.6525 99.5) (width 0.5) (layer "F.Cu") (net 1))
 (segment (start 230.6525 99.5) (end 230.965 99.8125) (width 0.5) (layer "F.Cu") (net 1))
 (segment (start 227.6 100.1) (end 228.2 99.5) (width 0.5) (layer "F.Cu") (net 1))
 (segment (start 231.3775 97.9875) (end 233.965 95.4) (width 0.5) (layer "F.Cu") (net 2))
 (segment (start 233.965 95.4) (end 233.965 93.9) (width 0.5) (layer "F.Cu") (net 2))
 (segment (start 230.965 97.9875) (end 231.3775 97.9875) (width 0.5) (layer "F.Cu") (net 2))
 (segment (start 227.6 97.9) (end 230.8775 97.9) (width 0.5) (layer "F.Cu") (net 2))
 (segment (start 230.8775 97.9) (end 230.965 97.9875) (width 0.5) (layer "F.Cu") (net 2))
 (segment (start 227.6 97.9) (end 227.6 96.425) (width 0.5) (layer "F.Cu") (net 2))
 (via (at 227.6 97.9) (size 0.6) (drill 0.3) (layers "F.Cu" "B.Cu") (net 2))
 (segment (start 226.2025 98) (end 227.5 98) (width 0.5) (layer "B.Cu") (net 2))
 (segment (start 227.5 98) (end 227.6 97.9) (width 0.5) (layer "B.Cu") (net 2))
 (segment (start 225.4025 98) (end 226.2025 98) (width 0.5) (layer "B.Cu") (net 2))
 (segment (start 226.33 99.67) (end 226.33 101.375) (width 0.5) (layer "F.Cu") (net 6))
 (via (at 226.33 99.67) (size 0.6) (drill 0.3) (layers "F.Cu" "B.Cu") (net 6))
 (segment (start 226.2 99.8) (end 224.6025 99.8) (width 0.5) (layer "B.Cu") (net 6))
 (segment (start 226.33 99.67) (end 226.2 99.8) (width 0.5) (layer "B.Cu") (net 6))
 (segment (start 225.06 96.425) (end 225.06 101.375) (width 0.5) (layer "F.Cu") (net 5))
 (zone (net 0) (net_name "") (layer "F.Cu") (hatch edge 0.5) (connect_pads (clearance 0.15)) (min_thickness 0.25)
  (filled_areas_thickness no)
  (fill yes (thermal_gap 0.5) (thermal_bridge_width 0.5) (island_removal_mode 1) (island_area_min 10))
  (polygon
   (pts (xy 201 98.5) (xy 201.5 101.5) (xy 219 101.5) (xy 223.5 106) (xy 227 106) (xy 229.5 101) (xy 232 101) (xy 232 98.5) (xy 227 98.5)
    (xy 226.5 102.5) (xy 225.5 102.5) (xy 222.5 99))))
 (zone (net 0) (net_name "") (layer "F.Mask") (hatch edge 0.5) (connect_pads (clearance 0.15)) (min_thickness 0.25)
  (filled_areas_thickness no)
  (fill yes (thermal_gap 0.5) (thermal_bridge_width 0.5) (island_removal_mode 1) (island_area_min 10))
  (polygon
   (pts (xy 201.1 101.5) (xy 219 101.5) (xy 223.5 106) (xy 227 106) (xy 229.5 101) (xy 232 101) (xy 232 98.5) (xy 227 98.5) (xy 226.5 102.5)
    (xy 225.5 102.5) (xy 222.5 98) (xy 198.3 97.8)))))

